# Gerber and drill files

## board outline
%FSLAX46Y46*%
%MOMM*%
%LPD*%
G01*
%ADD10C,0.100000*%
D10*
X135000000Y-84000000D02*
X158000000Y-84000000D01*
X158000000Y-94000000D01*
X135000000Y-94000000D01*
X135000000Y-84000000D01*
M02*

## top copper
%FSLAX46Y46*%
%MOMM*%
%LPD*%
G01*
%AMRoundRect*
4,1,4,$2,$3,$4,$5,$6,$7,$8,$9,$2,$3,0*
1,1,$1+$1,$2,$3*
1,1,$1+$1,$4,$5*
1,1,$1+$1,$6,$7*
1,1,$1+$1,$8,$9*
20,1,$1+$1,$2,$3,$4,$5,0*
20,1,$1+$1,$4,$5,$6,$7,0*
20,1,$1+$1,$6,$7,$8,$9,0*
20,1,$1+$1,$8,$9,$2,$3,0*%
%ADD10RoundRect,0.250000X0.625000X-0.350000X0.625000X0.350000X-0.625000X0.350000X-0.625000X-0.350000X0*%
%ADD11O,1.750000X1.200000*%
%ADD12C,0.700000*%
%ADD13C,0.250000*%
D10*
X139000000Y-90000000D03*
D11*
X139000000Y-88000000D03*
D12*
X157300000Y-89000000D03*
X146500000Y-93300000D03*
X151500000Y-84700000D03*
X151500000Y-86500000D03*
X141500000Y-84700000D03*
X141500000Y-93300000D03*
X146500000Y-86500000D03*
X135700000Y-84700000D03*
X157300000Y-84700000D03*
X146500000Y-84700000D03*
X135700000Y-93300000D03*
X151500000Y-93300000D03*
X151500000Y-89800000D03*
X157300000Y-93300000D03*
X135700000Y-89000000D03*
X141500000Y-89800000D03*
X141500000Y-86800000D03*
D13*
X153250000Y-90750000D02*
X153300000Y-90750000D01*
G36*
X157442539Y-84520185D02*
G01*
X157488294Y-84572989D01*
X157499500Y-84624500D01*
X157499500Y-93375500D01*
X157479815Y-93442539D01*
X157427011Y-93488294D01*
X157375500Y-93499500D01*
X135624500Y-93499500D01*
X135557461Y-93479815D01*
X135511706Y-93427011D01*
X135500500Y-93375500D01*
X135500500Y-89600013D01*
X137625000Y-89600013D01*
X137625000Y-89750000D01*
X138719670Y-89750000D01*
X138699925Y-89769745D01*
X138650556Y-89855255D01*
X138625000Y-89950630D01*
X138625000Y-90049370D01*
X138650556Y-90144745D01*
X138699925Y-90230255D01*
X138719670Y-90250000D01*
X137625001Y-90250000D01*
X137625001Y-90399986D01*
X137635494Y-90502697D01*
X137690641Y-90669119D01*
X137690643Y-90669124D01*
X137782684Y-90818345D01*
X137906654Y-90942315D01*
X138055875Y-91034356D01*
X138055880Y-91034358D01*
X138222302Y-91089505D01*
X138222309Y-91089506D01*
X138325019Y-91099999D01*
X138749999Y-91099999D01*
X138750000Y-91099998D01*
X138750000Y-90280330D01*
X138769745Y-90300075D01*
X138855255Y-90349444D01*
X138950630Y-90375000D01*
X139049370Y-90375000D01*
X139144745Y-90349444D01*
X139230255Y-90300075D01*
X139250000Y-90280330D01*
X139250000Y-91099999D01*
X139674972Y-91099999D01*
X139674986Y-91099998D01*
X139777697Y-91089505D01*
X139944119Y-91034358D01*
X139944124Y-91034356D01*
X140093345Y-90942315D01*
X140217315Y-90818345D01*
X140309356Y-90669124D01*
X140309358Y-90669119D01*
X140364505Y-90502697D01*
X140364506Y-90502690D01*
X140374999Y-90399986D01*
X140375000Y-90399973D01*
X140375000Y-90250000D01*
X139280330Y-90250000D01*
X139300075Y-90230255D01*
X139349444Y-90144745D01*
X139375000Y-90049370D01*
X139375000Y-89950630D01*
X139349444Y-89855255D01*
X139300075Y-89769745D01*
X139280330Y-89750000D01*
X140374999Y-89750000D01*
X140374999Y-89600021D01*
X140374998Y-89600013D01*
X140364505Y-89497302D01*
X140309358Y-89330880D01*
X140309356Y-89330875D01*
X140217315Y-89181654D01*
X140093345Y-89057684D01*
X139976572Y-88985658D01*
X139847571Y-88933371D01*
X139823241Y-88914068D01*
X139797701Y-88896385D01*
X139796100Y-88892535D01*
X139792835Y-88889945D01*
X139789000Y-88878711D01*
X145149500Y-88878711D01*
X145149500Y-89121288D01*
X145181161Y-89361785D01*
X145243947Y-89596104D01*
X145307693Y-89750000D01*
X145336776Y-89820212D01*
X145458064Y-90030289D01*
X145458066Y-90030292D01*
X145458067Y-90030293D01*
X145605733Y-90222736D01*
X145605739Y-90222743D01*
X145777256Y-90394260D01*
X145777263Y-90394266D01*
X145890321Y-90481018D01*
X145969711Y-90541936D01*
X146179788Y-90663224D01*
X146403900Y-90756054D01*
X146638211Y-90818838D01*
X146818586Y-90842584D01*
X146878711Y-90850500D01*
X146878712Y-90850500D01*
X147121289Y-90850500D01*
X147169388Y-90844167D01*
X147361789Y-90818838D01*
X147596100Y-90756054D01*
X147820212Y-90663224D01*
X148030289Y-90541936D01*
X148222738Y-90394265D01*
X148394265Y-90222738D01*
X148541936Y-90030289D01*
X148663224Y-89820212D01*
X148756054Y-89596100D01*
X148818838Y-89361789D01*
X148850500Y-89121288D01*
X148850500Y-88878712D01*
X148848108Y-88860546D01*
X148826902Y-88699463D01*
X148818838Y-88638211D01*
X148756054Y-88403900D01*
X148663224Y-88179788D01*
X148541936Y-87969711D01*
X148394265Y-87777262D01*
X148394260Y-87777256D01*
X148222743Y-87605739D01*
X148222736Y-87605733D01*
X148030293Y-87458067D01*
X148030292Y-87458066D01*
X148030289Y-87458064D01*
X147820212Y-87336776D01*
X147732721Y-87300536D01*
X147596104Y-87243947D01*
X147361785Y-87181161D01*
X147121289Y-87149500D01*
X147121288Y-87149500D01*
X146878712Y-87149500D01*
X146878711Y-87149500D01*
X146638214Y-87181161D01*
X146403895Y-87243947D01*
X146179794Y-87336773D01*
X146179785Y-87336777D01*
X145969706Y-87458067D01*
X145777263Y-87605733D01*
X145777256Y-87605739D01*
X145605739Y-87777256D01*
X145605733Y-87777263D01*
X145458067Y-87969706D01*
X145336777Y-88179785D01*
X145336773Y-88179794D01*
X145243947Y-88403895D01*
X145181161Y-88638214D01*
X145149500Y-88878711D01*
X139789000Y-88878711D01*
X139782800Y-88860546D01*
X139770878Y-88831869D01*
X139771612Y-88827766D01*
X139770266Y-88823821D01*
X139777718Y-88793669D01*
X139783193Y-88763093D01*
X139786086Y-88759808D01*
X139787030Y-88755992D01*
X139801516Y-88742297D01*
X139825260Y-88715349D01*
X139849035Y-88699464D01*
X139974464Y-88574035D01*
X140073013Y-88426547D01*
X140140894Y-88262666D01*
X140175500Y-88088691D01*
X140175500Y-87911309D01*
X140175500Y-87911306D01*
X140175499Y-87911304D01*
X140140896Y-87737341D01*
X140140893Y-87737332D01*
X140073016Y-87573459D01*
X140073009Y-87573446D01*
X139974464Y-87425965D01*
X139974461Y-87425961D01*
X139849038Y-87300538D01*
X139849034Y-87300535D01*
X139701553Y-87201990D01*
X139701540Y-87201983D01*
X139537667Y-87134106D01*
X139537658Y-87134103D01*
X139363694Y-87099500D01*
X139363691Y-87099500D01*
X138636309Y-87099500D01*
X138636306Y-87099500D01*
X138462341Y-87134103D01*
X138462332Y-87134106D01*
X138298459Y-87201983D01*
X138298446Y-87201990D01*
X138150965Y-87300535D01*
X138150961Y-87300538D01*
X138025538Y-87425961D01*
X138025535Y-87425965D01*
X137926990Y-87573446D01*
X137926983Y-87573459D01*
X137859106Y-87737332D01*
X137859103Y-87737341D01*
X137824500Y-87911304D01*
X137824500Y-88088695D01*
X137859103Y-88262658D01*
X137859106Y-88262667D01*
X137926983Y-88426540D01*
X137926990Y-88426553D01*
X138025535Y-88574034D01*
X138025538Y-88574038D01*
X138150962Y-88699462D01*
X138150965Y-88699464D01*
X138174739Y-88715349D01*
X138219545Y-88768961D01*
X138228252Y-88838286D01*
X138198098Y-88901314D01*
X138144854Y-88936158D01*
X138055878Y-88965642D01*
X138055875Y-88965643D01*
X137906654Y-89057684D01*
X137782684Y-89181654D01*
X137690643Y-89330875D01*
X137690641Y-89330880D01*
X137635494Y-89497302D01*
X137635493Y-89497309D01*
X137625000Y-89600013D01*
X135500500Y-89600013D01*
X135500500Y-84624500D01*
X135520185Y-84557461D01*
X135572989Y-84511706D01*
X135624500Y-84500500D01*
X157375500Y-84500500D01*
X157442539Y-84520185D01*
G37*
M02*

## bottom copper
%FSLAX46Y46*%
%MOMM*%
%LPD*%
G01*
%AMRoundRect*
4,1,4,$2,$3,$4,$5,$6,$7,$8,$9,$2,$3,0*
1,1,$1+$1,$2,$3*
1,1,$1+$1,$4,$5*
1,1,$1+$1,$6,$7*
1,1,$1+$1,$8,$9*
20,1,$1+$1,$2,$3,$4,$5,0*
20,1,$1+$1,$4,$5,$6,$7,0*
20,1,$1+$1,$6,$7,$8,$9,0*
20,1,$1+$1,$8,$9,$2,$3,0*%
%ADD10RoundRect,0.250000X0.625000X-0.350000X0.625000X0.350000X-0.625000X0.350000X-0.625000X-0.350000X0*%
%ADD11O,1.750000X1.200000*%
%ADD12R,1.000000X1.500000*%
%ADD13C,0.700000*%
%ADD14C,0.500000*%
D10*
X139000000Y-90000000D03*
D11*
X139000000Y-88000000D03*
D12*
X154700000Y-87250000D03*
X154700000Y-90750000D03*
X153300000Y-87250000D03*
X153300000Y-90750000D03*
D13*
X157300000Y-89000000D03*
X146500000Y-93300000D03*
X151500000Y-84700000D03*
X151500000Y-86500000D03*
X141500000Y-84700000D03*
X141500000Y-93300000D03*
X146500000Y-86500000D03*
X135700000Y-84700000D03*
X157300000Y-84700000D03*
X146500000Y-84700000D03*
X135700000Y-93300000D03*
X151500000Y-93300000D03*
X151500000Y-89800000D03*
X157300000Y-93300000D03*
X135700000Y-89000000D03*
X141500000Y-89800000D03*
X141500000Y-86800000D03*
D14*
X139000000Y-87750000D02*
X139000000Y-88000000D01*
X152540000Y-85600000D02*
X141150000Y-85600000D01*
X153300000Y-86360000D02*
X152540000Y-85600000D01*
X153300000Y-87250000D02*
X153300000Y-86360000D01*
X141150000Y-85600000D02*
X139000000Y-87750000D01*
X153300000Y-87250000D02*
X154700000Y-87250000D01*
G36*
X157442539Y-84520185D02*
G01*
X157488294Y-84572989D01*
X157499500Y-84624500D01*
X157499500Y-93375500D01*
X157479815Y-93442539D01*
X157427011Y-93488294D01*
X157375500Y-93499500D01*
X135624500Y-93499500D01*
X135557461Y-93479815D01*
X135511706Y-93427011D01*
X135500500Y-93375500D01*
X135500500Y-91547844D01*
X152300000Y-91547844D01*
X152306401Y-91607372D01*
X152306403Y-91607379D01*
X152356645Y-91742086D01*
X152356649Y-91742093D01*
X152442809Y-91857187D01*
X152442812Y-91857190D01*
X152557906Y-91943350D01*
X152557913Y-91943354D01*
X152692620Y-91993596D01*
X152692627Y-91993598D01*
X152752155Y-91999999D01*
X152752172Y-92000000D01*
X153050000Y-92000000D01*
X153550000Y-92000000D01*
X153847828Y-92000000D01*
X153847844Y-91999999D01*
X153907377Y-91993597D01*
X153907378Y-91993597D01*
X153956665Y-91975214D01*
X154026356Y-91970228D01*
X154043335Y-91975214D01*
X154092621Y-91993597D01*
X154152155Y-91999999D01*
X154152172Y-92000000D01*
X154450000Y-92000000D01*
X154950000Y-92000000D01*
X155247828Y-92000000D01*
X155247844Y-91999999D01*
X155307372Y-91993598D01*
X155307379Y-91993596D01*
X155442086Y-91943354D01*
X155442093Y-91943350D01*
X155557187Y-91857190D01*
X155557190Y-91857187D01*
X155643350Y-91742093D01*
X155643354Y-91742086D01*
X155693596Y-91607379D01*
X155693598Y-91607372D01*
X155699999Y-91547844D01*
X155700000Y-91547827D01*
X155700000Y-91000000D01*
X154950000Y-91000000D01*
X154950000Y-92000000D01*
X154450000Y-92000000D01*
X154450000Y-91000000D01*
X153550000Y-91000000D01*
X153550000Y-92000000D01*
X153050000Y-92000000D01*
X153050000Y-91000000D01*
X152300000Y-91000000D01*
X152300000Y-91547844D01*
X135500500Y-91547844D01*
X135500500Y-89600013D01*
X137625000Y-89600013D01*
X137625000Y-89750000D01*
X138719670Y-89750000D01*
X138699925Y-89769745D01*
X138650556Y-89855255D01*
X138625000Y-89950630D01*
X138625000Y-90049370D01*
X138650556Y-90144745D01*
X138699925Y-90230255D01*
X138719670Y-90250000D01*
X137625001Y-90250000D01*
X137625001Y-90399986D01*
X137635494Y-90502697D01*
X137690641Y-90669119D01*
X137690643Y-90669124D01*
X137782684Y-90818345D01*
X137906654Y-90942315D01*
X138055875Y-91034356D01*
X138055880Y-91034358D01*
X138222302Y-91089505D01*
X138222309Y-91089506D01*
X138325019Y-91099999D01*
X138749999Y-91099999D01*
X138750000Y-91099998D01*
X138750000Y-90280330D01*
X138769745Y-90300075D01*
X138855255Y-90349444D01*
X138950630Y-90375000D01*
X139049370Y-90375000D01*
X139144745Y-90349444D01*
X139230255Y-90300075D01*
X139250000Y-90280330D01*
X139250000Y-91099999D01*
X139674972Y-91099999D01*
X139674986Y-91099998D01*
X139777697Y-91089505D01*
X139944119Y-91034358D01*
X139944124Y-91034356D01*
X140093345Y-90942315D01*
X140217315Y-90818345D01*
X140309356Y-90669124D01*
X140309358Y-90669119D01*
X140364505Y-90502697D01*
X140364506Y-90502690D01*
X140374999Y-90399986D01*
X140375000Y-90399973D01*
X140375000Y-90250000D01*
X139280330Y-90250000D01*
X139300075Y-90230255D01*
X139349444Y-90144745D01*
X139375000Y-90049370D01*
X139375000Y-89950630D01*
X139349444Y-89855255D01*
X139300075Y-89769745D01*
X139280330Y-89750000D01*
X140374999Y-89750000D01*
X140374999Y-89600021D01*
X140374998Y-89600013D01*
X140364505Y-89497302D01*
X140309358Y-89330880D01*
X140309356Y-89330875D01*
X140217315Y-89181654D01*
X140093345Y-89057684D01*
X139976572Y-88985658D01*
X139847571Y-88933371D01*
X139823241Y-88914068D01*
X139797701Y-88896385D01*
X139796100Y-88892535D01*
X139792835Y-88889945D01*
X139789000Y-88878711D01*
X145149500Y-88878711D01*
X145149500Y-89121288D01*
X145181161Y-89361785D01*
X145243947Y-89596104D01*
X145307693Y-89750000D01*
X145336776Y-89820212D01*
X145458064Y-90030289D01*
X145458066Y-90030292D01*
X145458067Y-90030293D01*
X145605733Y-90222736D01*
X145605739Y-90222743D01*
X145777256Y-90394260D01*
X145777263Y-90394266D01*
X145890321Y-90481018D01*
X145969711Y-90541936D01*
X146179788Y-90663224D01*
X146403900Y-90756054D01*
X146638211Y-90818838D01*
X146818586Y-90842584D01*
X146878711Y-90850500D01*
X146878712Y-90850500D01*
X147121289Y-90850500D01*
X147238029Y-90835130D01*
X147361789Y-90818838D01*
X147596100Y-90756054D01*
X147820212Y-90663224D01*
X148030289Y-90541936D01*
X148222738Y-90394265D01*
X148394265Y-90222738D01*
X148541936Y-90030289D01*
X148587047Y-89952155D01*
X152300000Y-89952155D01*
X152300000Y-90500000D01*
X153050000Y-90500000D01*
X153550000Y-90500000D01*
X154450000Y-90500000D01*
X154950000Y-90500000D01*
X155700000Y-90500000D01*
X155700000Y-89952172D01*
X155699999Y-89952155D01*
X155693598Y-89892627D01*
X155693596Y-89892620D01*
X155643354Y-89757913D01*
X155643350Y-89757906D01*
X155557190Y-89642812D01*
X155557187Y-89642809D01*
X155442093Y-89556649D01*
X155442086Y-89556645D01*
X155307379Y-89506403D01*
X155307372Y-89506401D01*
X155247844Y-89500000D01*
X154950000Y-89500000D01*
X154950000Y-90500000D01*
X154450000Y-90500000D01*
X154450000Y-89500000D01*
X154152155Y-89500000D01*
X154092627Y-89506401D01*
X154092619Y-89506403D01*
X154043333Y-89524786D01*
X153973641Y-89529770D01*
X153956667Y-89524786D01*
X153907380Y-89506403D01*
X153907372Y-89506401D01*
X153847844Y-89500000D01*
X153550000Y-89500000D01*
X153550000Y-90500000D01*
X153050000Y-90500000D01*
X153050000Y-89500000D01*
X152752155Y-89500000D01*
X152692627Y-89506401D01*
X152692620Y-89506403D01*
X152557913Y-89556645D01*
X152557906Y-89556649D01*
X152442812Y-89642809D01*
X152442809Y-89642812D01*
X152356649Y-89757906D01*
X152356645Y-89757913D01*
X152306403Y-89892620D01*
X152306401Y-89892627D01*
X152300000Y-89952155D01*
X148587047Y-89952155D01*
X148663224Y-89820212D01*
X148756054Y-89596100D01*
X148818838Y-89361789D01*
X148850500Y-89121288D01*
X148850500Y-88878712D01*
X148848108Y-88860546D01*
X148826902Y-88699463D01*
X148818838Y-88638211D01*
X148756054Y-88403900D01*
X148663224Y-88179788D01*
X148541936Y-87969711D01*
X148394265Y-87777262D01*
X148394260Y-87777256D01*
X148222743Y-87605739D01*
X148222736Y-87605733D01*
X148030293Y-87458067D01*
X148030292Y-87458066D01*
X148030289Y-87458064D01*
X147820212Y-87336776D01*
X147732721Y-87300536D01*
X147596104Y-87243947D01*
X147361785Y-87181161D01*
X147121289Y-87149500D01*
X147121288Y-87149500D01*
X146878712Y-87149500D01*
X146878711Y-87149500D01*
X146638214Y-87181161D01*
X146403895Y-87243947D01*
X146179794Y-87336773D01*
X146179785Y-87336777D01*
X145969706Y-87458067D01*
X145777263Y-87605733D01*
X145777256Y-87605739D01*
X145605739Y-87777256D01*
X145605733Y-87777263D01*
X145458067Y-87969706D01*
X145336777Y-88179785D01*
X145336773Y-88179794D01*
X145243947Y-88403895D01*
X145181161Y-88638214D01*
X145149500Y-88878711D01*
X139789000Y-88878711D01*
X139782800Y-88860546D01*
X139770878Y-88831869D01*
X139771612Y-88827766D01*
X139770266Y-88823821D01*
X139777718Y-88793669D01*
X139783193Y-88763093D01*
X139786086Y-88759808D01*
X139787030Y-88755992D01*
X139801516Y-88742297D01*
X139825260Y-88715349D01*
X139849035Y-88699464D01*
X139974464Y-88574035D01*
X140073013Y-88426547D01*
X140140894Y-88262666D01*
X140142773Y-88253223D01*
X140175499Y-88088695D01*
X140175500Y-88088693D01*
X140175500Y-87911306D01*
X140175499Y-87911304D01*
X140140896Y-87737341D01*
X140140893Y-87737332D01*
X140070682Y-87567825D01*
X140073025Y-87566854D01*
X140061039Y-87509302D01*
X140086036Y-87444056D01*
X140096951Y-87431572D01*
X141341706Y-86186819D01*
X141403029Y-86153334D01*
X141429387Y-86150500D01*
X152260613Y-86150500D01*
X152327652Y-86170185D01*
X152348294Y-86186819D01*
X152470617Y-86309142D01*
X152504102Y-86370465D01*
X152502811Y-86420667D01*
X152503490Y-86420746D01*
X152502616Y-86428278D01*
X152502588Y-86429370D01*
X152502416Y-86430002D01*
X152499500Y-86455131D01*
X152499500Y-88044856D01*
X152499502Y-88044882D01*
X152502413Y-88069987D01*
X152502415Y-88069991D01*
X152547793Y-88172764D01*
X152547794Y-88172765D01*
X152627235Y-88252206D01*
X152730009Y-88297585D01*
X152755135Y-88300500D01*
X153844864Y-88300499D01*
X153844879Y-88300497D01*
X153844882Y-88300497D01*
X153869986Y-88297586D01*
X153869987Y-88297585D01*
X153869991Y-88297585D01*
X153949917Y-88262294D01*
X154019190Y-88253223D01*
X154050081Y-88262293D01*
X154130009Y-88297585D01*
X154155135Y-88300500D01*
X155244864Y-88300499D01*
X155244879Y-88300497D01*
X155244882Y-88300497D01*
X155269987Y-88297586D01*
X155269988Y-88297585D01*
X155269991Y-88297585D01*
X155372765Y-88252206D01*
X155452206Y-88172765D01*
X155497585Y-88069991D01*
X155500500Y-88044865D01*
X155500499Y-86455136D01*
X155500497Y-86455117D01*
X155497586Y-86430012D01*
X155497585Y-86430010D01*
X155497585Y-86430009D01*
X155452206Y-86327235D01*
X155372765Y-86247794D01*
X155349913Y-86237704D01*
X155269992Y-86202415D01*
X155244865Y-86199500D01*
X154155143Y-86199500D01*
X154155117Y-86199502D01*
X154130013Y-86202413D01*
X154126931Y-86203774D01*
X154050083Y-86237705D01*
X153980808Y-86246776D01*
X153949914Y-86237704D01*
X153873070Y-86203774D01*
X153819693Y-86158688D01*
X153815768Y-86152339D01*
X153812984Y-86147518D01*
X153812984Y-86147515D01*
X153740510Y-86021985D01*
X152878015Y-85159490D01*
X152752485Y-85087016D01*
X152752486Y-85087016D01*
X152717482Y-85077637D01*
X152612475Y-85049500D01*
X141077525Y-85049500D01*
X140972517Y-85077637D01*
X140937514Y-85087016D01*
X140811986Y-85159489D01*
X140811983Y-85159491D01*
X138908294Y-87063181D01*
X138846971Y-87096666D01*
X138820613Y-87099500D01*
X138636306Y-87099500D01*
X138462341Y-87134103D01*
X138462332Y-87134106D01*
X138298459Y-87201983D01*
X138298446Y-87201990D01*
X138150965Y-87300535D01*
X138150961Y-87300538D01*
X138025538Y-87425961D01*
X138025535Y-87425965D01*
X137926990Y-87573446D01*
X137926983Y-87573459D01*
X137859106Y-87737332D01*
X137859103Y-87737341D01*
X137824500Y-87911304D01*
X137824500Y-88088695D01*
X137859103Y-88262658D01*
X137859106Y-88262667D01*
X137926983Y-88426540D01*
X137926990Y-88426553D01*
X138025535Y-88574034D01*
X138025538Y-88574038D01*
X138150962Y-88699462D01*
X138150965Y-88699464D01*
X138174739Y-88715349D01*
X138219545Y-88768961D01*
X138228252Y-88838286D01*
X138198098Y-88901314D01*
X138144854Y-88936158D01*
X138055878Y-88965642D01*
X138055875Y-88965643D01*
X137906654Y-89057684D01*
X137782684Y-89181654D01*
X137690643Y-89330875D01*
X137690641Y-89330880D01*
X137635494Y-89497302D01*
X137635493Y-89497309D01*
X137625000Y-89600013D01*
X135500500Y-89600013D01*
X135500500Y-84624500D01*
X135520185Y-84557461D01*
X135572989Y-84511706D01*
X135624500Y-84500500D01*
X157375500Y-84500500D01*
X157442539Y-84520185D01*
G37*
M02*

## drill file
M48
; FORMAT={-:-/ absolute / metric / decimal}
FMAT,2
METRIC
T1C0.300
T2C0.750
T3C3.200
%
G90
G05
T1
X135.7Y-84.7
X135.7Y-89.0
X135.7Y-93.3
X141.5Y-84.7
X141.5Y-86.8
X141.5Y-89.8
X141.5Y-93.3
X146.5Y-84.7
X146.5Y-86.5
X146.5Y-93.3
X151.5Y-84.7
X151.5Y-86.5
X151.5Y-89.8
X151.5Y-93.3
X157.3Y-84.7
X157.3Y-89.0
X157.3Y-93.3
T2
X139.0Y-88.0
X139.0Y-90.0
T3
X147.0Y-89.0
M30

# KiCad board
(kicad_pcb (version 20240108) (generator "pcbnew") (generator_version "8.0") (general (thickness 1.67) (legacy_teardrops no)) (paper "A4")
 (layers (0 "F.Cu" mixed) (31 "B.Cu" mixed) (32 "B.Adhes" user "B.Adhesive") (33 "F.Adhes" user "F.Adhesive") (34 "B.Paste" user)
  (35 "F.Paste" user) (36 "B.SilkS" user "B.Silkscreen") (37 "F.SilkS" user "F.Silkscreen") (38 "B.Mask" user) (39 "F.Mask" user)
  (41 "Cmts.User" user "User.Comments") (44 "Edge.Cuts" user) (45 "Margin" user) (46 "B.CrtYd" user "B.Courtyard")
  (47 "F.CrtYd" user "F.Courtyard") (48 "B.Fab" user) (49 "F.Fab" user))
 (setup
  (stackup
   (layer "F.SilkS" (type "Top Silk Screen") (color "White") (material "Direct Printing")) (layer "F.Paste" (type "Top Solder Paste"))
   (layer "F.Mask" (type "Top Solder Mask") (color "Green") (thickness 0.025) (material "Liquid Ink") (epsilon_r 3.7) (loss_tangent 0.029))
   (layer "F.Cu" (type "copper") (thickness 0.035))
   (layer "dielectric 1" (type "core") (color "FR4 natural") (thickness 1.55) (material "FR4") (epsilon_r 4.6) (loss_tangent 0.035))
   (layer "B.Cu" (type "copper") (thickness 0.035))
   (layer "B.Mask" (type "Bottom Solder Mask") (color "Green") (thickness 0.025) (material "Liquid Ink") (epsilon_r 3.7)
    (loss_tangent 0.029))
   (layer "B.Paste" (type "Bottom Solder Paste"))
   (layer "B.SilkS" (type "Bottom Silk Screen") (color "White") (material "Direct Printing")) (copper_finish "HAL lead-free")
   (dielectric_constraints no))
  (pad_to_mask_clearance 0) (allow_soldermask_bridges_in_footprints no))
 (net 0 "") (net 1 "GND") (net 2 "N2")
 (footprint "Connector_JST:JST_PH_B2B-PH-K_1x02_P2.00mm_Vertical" (layer "F.Cu") (at 139 90 90)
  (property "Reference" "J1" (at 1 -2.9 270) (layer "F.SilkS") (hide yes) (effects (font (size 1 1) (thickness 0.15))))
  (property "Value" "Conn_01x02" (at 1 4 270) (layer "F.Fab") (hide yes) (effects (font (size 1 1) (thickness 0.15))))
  (pad "1" thru_hole roundrect (at 0 0 90) (size 1.2 1.75) (drill 0.75) (layers "*.Cu" "*.Mask") (remove_unused_layers no)
   (roundrect_rratio 0.208333) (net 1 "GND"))
  (pad "2" thru_hole oval (at 2 0 90) (size 1.2 1.75) (drill 0.75) (layers "*.Cu" "*.Mask") (remove_unused_layers no) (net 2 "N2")))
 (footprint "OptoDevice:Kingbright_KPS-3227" (layer "B.Cu") (at 154 89 180)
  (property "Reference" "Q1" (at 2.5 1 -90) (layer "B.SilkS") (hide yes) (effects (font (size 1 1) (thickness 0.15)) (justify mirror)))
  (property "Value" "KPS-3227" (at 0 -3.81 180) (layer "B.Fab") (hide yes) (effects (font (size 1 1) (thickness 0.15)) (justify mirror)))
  (pad "1" smd rect (at -0.7 1.75 180) (size 1 1.5) (layers "B.Cu" "B.Paste" "B.Mask") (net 2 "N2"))
  (pad "2" smd rect (at -0.7 -1.75 180) (size 1 1.5) (layers "B.Cu" "B.Paste" "B.Mask") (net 1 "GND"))
  (pad "3" smd rect (at 0.7 1.75 180) (size 1 1.5) (layers "B.Cu" "B.Paste" "B.Mask") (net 2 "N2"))
  (pad "4" smd rect (at 0.7 -1.75 180) (size 1 1.5) (layers "B.Cu" "B.Paste" "B.Mask") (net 1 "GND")))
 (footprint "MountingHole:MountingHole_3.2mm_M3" (layer "B.Cu") (at 147 89 -90)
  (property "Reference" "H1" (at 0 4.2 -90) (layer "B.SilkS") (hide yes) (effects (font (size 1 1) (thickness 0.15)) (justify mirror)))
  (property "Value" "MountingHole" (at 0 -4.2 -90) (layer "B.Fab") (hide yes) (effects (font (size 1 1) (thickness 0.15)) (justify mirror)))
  (pad "" np_thru_hole circle (at 0 0 270) (size 3.2 3.2) (drill 3.2) (layers "*.Cu" "*.Mask")))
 (gr_rect (start 135 84) (end 158 94) (stroke (width 0.1) (type default)) (fill none) (layer "Edge.Cuts"))
 (segment (start 139 87.75) (end 139 88) (width 0.5) (layer "B.Cu") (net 2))
 (segment (start 152.54 85.6) (end 141.15 85.6) (width 0.5) (layer "B.Cu") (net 2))
 (segment (start 153.3 86.36) (end 152.54 85.6) (width 0.5) (layer "B.Cu") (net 2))
 (segment (start 153.3 87.25) (end 153.3 86.36) (width 0.5) (layer "B.Cu") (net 2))
 (segment (start 141.15 85.6) (end 139 87.75) (width 0.5) (layer "B.Cu") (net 2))
 (segment (start 153.3 87.25) (end 154.7 87.25) (width 0.5) (layer "B.Cu") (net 2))
 (segment (start 153.25 90.75) (end 153.3 90.75) (width 0.25) (layer "F.Cu") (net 1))
 (via (at 157.3 89) (size 0.7) (drill 0.3) (layers "F.Cu" "B.Cu") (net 1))
 (via (at 146.5 93.3) (size 0.7) (drill 0.3) (layers "F.Cu" "B.Cu") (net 1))
 (via (at 151.5 84.7) (size 0.7) (drill 0.3) (layers "F.Cu" "B.Cu") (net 1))
 (via (at 151.5 86.5) (size 0.7) (drill 0.3) (layers "F.Cu" "B.Cu") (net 1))
 (via (at 141.5 84.7) (size 0.7) (drill 0.3) (layers "F.Cu" "B.Cu") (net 1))
 (via (at 141.5 93.3) (size 0.7) (drill 0.3) (layers "F.Cu" "B.Cu") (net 1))
 (via (at 146.5 86.5) (size 0.7) (drill 0.3) (layers "F.Cu" "B.Cu") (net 1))
 (via (at 135.7 84.7) (size 0.7) (drill 0.3) (layers "F.Cu" "B.Cu") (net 1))
 (via (at 157.3 84.7) (size 0.7) (drill 0.3) (layers "F.Cu" "B.Cu") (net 1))
 (via (at 146.5 84.7) (size 0.7) (drill 0.3) (layers "F.Cu" "B.Cu") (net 1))
 (via (at 135.7 93.3) (size 0.7) (drill 0.3) (layers "F.Cu" "B.Cu") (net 1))
 (via (at 151.5 93.3) (size 0.7) (drill 0.3) (layers "F.Cu" "B.Cu") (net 1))
 (via (at 151.5 89.8) (size 0.7) (drill 0.3) (layers "F.Cu" "B.Cu") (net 1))
 (via (at 157.3 93.3) (size 0.7) (drill 0.3) (layers "F.Cu" "B.Cu") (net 1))
 (via (at 135.7 89) (size 0.7) (drill 0.3) (layers "F.Cu" "B.Cu") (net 1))
 (via (at 141.5 89.8) (size 0.7) (drill 0.3) (layers "F.Cu" "B.Cu") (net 1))
 (via (at 141.5 86.8) (size 0.7) (drill 0.3) (layers "F.Cu" "B.Cu") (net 1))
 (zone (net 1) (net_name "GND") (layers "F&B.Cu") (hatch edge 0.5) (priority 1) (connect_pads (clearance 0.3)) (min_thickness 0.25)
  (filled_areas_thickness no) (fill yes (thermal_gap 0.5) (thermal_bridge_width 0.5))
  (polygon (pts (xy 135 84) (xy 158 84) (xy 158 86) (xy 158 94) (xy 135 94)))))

